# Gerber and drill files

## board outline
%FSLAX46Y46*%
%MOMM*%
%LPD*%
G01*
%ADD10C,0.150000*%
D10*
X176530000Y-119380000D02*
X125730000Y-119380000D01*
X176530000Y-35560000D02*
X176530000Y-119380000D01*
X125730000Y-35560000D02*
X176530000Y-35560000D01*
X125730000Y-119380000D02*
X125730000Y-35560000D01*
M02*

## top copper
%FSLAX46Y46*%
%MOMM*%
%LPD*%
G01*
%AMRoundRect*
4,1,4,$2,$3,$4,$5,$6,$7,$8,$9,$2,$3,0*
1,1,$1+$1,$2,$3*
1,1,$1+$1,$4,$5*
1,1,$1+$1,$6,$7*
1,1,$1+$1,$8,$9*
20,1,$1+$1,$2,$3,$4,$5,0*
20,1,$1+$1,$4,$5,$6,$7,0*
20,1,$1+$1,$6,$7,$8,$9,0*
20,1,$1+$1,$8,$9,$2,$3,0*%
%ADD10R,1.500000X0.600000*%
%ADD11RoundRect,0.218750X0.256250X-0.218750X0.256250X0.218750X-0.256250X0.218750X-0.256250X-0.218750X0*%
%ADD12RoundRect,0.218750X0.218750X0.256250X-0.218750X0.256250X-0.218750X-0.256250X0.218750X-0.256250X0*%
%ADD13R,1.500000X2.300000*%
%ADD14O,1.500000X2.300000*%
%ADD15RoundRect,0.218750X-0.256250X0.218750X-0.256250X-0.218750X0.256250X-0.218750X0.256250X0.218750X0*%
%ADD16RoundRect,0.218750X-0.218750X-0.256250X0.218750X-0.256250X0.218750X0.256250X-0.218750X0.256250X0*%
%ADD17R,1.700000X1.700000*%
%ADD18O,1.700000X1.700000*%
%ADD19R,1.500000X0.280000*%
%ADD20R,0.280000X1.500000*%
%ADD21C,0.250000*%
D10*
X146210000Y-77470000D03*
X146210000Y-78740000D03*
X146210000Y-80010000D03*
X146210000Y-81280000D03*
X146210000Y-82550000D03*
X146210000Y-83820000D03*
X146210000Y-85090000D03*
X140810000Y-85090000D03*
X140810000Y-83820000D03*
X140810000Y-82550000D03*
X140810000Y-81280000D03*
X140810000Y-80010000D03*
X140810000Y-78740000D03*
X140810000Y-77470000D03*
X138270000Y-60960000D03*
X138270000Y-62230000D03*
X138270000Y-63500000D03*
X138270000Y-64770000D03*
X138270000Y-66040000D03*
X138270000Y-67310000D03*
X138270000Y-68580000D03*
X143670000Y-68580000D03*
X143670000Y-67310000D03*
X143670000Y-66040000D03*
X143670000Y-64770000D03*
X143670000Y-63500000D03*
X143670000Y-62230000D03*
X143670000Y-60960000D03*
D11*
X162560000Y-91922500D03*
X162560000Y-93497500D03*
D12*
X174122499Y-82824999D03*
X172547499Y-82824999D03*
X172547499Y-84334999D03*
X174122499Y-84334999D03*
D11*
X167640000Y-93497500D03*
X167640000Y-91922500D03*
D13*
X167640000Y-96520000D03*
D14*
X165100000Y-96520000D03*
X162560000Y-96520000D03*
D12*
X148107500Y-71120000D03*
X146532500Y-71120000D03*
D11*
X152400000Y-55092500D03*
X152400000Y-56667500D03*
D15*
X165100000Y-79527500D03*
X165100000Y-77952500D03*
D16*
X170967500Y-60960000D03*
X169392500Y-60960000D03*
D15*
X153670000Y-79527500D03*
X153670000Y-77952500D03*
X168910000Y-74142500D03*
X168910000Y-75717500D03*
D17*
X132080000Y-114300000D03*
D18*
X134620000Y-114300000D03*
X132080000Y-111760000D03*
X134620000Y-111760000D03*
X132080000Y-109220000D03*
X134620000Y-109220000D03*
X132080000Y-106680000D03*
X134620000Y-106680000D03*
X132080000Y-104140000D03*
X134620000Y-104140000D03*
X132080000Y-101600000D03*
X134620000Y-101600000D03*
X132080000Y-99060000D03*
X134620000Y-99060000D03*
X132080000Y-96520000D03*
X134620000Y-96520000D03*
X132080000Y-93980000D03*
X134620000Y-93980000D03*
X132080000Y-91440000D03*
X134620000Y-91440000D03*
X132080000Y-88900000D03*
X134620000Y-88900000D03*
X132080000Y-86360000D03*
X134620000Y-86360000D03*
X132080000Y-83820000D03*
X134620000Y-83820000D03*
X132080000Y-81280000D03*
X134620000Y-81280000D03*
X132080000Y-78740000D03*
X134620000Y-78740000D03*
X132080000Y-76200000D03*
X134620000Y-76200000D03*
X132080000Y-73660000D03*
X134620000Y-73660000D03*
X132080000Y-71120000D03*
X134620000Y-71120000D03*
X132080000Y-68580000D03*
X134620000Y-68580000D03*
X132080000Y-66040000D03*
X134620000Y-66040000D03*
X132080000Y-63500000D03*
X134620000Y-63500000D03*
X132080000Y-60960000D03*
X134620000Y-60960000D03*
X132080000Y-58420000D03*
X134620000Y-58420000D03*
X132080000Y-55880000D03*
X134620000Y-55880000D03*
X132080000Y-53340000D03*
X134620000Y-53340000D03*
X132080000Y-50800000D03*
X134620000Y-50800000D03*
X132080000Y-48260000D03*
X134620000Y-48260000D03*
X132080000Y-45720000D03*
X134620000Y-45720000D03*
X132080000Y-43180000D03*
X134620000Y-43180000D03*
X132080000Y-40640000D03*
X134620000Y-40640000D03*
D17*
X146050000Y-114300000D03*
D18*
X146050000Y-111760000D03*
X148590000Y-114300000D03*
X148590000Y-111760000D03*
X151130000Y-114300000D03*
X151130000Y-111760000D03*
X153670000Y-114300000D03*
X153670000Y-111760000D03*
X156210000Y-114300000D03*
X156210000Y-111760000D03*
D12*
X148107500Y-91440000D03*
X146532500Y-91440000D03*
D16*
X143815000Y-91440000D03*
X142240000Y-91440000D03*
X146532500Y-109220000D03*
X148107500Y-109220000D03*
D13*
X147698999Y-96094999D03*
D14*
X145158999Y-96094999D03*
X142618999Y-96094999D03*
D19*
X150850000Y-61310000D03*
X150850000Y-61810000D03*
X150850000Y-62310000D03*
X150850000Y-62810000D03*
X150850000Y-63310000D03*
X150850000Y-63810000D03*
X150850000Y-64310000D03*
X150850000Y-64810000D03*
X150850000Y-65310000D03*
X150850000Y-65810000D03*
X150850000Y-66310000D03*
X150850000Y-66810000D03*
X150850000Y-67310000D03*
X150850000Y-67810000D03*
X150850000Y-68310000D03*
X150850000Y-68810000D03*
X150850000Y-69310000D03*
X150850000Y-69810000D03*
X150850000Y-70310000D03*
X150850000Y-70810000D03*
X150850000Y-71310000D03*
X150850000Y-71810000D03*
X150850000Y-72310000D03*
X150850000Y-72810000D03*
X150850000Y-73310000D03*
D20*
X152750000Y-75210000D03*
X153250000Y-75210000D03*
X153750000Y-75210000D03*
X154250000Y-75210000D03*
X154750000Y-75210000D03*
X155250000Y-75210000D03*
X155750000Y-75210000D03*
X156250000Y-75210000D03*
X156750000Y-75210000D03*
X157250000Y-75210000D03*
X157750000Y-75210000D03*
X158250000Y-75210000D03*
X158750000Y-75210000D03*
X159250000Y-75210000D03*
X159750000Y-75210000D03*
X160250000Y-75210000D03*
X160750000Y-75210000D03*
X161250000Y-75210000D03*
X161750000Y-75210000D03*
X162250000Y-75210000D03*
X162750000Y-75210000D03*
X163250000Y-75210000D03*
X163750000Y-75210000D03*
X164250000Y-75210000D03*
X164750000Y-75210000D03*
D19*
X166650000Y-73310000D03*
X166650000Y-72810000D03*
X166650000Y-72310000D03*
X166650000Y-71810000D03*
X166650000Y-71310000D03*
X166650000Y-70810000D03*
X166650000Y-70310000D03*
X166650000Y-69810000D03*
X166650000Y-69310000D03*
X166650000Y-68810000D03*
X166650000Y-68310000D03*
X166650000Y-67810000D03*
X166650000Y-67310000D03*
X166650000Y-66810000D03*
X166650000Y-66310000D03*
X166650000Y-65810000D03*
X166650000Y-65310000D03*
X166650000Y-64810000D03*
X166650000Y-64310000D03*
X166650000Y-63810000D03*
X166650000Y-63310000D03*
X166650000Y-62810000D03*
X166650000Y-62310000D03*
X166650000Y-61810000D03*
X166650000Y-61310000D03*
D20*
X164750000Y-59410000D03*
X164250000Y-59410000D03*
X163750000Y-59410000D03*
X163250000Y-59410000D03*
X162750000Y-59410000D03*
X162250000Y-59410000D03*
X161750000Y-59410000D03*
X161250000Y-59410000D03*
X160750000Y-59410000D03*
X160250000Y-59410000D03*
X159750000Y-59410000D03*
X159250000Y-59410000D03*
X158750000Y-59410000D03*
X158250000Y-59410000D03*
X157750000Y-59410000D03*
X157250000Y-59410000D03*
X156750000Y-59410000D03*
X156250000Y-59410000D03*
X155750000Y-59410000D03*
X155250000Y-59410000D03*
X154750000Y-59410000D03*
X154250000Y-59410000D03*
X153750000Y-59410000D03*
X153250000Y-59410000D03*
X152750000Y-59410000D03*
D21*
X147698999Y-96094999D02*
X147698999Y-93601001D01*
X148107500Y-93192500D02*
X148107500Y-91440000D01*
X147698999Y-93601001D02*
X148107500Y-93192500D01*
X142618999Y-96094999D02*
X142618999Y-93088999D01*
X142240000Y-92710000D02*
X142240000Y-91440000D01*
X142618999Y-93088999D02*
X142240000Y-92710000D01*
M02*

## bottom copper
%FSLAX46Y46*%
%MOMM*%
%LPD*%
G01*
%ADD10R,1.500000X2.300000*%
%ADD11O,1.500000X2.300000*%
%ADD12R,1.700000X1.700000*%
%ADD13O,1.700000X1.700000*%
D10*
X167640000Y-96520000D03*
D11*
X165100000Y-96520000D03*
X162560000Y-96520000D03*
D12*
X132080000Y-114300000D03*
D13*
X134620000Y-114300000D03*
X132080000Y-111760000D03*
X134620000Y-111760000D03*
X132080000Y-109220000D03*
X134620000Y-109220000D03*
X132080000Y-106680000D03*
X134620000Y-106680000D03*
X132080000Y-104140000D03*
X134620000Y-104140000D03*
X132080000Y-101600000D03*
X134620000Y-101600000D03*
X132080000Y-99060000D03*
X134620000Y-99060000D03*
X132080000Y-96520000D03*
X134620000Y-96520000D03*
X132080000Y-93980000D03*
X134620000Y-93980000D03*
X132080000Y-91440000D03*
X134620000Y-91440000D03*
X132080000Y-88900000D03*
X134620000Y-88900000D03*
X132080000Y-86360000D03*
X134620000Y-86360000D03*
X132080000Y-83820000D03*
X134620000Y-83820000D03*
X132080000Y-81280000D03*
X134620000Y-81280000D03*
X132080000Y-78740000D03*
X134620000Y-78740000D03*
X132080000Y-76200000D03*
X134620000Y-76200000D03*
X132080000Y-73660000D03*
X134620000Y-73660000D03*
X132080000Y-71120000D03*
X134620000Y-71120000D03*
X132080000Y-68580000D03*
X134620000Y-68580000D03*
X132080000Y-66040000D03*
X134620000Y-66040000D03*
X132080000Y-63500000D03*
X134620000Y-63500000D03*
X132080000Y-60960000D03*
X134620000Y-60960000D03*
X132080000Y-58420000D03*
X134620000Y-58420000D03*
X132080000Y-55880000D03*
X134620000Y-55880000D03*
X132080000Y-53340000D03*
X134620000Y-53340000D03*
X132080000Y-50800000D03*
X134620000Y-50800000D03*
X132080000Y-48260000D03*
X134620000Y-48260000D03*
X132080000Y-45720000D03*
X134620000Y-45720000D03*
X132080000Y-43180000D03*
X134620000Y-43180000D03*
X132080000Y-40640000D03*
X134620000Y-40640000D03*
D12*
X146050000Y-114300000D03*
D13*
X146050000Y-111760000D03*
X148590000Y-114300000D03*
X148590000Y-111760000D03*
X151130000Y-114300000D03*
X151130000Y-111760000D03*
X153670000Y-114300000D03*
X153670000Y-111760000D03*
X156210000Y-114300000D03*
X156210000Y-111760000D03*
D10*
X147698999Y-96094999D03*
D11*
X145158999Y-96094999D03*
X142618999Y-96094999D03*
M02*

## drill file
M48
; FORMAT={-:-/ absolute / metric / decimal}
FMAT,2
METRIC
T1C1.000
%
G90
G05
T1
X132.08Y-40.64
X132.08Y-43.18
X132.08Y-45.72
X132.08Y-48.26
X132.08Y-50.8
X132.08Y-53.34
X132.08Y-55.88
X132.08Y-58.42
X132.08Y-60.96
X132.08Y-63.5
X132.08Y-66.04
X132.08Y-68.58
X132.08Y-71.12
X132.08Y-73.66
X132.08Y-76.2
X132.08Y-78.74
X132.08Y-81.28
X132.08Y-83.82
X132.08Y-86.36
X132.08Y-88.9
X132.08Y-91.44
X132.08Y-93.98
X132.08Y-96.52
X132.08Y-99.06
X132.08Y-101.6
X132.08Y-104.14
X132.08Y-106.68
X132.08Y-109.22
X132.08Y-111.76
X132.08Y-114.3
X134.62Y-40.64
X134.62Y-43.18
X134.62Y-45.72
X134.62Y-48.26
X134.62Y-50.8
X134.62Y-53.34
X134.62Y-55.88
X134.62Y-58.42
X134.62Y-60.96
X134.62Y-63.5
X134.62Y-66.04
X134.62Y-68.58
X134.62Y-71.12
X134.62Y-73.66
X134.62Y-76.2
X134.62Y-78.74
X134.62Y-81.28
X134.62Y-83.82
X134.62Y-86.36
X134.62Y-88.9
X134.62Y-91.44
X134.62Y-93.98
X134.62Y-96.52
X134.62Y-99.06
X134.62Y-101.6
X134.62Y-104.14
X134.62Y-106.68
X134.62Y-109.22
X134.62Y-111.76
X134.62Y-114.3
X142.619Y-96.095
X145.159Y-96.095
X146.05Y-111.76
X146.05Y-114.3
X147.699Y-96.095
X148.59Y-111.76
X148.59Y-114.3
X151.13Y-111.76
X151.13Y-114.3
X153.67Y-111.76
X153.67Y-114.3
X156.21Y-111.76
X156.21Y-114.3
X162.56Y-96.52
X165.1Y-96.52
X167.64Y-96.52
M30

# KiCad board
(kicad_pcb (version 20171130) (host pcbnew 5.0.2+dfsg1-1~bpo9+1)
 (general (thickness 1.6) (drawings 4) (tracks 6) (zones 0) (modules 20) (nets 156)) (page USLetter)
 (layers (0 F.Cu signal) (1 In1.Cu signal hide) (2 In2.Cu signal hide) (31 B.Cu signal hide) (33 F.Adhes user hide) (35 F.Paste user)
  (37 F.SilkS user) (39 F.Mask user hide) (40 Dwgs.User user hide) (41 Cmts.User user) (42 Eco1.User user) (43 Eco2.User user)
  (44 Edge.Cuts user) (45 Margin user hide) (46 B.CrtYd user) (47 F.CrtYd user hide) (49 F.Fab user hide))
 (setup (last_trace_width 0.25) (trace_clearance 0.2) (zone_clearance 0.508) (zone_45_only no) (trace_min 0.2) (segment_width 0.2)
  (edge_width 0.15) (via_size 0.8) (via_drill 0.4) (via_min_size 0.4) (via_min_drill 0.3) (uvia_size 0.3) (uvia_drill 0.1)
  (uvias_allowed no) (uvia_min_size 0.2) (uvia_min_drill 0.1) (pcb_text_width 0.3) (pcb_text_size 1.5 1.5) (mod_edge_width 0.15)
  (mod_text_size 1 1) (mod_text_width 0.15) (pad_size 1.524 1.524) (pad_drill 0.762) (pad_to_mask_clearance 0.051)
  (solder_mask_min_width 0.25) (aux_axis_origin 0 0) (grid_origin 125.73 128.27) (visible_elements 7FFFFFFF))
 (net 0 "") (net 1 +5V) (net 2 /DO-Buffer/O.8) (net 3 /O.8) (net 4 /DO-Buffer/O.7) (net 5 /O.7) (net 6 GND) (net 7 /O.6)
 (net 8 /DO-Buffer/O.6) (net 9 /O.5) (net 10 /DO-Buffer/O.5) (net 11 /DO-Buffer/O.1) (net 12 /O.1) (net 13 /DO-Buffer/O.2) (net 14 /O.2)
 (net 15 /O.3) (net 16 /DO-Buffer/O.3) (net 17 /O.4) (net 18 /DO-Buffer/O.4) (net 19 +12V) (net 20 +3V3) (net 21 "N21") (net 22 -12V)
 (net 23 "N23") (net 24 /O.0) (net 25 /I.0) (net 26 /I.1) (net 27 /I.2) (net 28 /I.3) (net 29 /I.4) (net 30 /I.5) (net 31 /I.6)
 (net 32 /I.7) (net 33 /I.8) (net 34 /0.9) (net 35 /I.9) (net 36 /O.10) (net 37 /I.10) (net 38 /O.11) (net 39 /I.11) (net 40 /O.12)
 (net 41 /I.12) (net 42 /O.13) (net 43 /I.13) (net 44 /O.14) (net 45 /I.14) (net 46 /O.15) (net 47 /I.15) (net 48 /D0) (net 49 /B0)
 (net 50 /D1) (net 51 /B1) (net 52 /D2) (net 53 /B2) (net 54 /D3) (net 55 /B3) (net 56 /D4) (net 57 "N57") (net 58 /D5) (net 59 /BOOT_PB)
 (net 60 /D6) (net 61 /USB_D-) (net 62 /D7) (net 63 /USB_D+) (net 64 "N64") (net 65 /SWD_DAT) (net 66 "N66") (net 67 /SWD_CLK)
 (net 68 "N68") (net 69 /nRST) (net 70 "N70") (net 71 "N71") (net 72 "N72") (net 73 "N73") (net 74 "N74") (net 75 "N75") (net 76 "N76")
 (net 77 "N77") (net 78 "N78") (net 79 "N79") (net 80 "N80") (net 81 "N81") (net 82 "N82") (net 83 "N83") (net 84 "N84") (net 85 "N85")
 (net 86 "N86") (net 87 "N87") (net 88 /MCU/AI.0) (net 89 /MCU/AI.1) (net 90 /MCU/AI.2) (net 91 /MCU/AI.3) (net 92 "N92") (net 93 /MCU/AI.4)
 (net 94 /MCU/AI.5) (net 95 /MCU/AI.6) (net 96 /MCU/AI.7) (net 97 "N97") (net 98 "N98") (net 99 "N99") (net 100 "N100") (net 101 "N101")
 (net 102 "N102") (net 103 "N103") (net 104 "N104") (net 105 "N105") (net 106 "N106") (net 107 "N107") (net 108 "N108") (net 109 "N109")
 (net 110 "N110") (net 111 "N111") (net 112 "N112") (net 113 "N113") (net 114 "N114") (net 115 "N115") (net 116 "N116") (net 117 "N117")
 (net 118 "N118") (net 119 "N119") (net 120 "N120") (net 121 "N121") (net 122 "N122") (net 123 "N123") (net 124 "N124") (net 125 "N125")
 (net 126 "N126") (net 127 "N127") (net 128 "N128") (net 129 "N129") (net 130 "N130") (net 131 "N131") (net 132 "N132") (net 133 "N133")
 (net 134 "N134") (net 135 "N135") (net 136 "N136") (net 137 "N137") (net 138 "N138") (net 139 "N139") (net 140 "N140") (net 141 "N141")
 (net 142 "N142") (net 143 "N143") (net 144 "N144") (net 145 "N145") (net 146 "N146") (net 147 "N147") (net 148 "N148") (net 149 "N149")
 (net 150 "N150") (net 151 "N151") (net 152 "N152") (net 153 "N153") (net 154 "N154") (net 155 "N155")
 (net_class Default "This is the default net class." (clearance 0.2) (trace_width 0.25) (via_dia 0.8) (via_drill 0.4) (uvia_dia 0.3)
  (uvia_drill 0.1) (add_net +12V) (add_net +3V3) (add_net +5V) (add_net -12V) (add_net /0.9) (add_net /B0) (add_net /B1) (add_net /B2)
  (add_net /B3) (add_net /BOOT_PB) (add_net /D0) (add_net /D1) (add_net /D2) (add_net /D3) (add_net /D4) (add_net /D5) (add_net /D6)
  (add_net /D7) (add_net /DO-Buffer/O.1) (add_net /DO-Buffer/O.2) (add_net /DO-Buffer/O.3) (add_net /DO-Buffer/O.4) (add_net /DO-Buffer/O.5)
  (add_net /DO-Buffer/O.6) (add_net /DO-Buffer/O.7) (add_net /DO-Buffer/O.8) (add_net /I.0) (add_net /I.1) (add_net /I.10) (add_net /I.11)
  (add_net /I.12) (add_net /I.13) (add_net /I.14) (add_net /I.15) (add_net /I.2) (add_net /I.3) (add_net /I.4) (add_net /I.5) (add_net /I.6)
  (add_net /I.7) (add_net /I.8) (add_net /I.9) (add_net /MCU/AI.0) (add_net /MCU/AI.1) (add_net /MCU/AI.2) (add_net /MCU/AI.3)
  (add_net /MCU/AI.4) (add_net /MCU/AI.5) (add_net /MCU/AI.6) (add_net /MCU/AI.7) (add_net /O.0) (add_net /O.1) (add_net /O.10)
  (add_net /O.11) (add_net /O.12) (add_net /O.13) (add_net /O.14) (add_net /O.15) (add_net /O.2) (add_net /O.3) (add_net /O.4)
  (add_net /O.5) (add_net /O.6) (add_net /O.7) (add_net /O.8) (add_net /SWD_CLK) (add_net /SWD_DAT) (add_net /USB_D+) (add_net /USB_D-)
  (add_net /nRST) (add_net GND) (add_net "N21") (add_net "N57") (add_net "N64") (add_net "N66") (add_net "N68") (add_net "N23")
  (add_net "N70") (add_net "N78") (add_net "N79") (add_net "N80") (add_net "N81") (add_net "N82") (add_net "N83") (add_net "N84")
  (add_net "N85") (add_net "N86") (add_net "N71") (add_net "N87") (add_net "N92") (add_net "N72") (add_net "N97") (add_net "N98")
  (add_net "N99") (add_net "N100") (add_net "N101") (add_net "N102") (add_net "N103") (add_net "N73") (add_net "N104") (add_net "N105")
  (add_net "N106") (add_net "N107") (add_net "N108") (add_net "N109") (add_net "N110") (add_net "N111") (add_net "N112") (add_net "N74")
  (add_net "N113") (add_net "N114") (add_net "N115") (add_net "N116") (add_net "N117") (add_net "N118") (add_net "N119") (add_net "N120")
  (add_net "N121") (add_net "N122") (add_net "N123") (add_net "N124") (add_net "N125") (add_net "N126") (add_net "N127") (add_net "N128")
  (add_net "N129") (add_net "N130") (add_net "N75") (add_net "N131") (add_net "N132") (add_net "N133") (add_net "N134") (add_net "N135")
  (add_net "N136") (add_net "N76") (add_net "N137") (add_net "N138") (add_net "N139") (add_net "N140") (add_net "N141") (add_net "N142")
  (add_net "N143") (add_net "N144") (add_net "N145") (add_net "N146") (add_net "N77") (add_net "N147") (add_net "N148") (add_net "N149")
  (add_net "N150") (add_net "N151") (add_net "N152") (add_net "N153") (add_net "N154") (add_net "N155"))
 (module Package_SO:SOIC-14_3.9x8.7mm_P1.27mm (layer F.Cu) (at 143.51 81.28)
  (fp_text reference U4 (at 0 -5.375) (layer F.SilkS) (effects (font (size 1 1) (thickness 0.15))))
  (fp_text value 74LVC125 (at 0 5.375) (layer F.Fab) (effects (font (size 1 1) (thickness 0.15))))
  (pad 14 smd rect (at 2.7 -3.81) (size 1.5 0.6) (layers F.Cu F.Paste F.Mask) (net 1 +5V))
  (pad 13 smd rect (at 2.7 -2.54) (size 1.5 0.6) (layers F.Cu F.Paste F.Mask) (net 1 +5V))
  (pad 12 smd rect (at 2.7 -1.27) (size 1.5 0.6) (layers F.Cu F.Paste F.Mask) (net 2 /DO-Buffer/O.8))
  (pad 11 smd rect (at 2.7 0) (size 1.5 0.6) (layers F.Cu F.Paste F.Mask) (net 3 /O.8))
  (pad 10 smd rect (at 2.7 1.27) (size 1.5 0.6) (layers F.Cu F.Paste F.Mask) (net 1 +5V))
  (pad 9 smd rect (at 2.7 2.54) (size 1.5 0.6) (layers F.Cu F.Paste F.Mask) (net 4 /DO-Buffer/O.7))
  (pad 8 smd rect (at 2.7 3.81) (size 1.5 0.6) (layers F.Cu F.Paste F.Mask) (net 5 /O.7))
  (pad 7 smd rect (at -2.7 3.81) (size 1.5 0.6) (layers F.Cu F.Paste F.Mask) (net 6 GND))
  (pad 6 smd rect (at -2.7 2.54) (size 1.5 0.6) (layers F.Cu F.Paste F.Mask) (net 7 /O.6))
  (pad 5 smd rect (at -2.7 1.27) (size 1.5 0.6) (layers F.Cu F.Paste F.Mask) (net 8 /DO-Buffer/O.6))
  (pad 4 smd rect (at -2.7 0) (size 1.5 0.6) (layers F.Cu F.Paste F.Mask) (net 1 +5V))
  (pad 3 smd rect (at -2.7 -1.27) (size 1.5 0.6) (layers F.Cu F.Paste F.Mask) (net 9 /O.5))
  (pad 2 smd rect (at -2.7 -2.54) (size 1.5 0.6) (layers F.Cu F.Paste F.Mask) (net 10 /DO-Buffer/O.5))
  (pad 1 smd rect (at -2.7 -3.81) (size 1.5 0.6) (layers F.Cu F.Paste F.Mask) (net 1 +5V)))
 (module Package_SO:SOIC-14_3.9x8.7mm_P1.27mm (layer F.Cu) (at 140.97 64.77)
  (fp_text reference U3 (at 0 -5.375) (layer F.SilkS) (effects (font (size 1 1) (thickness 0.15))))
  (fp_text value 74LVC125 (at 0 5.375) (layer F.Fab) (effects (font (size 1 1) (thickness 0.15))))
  (pad 1 smd rect (at -2.7 -3.81) (size 1.5 0.6) (layers F.Cu F.Paste F.Mask) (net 1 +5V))
  (pad 2 smd rect (at -2.7 -2.54) (size 1.5 0.6) (layers F.Cu F.Paste F.Mask) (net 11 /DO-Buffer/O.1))
  (pad 3 smd rect (at -2.7 -1.27) (size 1.5 0.6) (layers F.Cu F.Paste F.Mask) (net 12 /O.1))
  (pad 4 smd rect (at -2.7 0) (size 1.5 0.6) (layers F.Cu F.Paste F.Mask) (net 1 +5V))
  (pad 5 smd rect (at -2.7 1.27) (size 1.5 0.6) (layers F.Cu F.Paste F.Mask) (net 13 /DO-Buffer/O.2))
  (pad 6 smd rect (at -2.7 2.54) (size 1.5 0.6) (layers F.Cu F.Paste F.Mask) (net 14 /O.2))
  (pad 7 smd rect (at -2.7 3.81) (size 1.5 0.6) (layers F.Cu F.Paste F.Mask) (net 6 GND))
  (pad 8 smd rect (at 2.7 3.81) (size 1.5 0.6) (layers F.Cu F.Paste F.Mask) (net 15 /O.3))
  (pad 9 smd rect (at 2.7 2.54) (size 1.5 0.6) (layers F.Cu F.Paste F.Mask) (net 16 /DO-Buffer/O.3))
  (pad 10 smd rect (at 2.7 1.27) (size 1.5 0.6) (layers F.Cu F.Paste F.Mask) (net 1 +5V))
  (pad 11 smd rect (at 2.7 0) (size 1.5 0.6) (layers F.Cu F.Paste F.Mask) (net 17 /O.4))
  (pad 12 smd rect (at 2.7 -1.27) (size 1.5 0.6) (layers F.Cu F.Paste F.Mask) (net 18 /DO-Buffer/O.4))
  (pad 13 smd rect (at 2.7 -2.54) (size 1.5 0.6) (layers F.Cu F.Paste F.Mask) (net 1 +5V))
  (pad 14 smd rect (at 2.7 -3.81) (size 1.5 0.6) (layers F.Cu F.Paste F.Mask) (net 1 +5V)))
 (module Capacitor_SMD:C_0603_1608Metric (layer F.Cu) (at 162.56 92.71 90)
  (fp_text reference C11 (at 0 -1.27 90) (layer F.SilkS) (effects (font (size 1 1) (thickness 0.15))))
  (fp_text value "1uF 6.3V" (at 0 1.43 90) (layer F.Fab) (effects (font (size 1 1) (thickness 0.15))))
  (pad 2 smd roundrect (at 0.7875 0 90) (size 0.875 0.95) (layers F.Cu F.Paste F.Mask) (roundrect_rratio 0.25) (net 6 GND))
  (pad 1 smd roundrect (at -0.7875 0 90) (size 0.875 0.95) (layers F.Cu F.Paste F.Mask) (roundrect_rratio 0.25) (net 1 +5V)))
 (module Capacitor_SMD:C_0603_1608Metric (layer F.Cu) (at 173.334999 82.824999 180)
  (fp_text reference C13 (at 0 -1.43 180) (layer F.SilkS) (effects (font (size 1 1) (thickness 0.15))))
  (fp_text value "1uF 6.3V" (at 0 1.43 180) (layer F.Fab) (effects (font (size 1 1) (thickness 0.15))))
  (pad 1 smd roundrect (at -0.7875 0 180) (size 0.875 0.95) (layers F.Cu F.Paste F.Mask) (roundrect_rratio 0.25) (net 1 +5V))
  (pad 2 smd roundrect (at 0.7875 0 180) (size 0.875 0.95) (layers F.Cu F.Paste F.Mask) (roundrect_rratio 0.25) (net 6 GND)))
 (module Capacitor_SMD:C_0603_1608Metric (layer F.Cu) (at 173.334999 84.334999 180)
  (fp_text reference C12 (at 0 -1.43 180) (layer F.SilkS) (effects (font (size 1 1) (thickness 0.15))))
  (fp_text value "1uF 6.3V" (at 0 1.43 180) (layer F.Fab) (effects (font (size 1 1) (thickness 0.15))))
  (pad 2 smd roundrect (at 0.7875 0 180) (size 0.875 0.95) (layers F.Cu F.Paste F.Mask) (roundrect_rratio 0.25) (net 6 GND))
  (pad 1 smd roundrect (at -0.7875 0 180) (size 0.875 0.95) (layers F.Cu F.Paste F.Mask) (roundrect_rratio 0.25) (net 1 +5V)))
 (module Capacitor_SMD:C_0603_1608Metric (layer F.Cu) (at 167.64 92.71 90)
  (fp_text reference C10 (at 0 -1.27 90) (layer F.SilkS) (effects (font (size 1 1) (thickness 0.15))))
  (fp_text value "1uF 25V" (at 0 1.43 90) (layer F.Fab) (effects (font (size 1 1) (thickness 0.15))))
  (pad 1 smd roundrect (at -0.7875 0 90) (size 0.875 0.95) (layers F.Cu F.Paste F.Mask) (roundrect_rratio 0.25) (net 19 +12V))
  (pad 2 smd roundrect (at 0.7875 0 90) (size 0.875 0.95) (layers F.Cu F.Paste F.Mask) (roundrect_rratio 0.25) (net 6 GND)))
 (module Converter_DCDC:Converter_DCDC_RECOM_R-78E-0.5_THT (layer F.Cu) (at 167.64 96.52 180)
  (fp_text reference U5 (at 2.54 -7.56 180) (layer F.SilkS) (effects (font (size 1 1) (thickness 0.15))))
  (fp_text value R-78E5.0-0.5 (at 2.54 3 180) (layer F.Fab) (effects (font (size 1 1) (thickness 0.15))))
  (pad 1 thru_hole rect (at 0 0 180) (size 1.5 2.3) (drill 1) (layers *.Cu *.Mask) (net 19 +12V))
  (pad 2 thru_hole oval (at 2.54 0 180) (size 1.5 2.3) (drill 1) (layers *.Cu *.Mask) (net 6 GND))
  (pad 3 thru_hole oval (at 5.08 0 180) (size 1.5 2.3) (drill 1) (layers *.Cu *.Mask) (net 1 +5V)))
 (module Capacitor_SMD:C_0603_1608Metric (layer F.Cu) (at 147.32 71.12 180)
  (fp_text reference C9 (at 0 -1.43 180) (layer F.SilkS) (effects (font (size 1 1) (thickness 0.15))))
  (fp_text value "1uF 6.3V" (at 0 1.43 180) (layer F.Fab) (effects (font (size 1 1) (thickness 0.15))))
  (pad 1 smd roundrect (at -0.7875 0 180) (size 0.875 0.95) (layers F.Cu F.Paste F.Mask) (roundrect_rratio 0.25) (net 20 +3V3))
  (pad 2 smd roundrect (at 0.7875 0 180) (size 0.875 0.95) (layers F.Cu F.Paste F.Mask) (roundrect_rratio 0.25) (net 6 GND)))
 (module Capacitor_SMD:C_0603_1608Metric (layer F.Cu) (at 152.4 55.88 90)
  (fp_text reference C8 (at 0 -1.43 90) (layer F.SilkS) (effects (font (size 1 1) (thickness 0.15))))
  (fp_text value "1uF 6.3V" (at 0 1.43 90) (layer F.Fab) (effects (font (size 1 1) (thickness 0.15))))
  (pad 2 smd roundrect (at 0.7875 0 90) (size 0.875 0.95) (layers F.Cu F.Paste F.Mask) (roundrect_rratio 0.25) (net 6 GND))
  (pad 1 smd roundrect (at -0.7875 0 90) (size 0.875 0.95) (layers F.Cu F.Paste F.Mask) (roundrect_rratio 0.25) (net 20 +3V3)))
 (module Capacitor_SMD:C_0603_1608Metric (layer F.Cu) (at 165.1 78.74 270)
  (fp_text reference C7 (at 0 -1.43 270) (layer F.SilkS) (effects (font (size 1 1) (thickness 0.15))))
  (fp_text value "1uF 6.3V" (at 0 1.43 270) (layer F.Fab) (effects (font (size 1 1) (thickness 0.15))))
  (pad 2 smd roundrect (at 0.7875 0 270) (size 0.875 0.95) (layers F.Cu F.Paste F.Mask) (roundrect_rratio 0.25) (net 6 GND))
  (pad 1 smd roundrect (at -0.7875 0 270) (size 0.875 0.95) (layers F.Cu F.Paste F.Mask) (roundrect_rratio 0.25) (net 20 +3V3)))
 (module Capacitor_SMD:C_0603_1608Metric (layer F.Cu) (at 170.18 60.96)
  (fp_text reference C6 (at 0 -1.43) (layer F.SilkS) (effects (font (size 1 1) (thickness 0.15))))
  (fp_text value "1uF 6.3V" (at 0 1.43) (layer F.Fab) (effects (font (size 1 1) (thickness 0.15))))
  (pad 2 smd roundrect (at 0.7875 0) (size 0.875 0.95) (layers F.Cu F.Paste F.Mask) (roundrect_rratio 0.25) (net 6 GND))
  (pad 1 smd roundrect (at -0.7875 0) (size 0.875 0.95) (layers F.Cu F.Paste F.Mask) (roundrect_rratio 0.25) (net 20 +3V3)))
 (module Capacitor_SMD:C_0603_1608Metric (layer F.Cu) (at 153.67 78.74 270)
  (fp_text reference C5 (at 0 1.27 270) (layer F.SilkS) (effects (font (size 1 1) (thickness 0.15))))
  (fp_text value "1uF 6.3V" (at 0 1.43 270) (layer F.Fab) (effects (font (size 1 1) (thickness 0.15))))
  (pad 2 smd roundrect (at 0.7875 0 270) (size 0.875 0.95) (layers F.Cu F.Paste F.Mask) (roundrect_rratio 0.25) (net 6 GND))
  (pad 1 smd roundrect (at -0.7875 0 270) (size 0.875 0.95) (layers F.Cu F.Paste F.Mask) (roundrect_rratio 0.25) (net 20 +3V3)))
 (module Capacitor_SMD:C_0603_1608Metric (layer F.Cu) (at 168.91 74.93 270)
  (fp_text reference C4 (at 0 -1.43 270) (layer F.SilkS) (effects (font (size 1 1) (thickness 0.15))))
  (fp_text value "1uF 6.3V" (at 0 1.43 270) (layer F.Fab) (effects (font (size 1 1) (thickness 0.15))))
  (pad 1 smd roundrect (at -0.7875 0 270) (size 0.875 0.95) (layers F.Cu F.Paste F.Mask) (roundrect_rratio 0.25) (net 20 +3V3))
  (pad 2 smd roundrect (at 0.7875 0 270) (size 0.875 0.95) (layers F.Cu F.Paste F.Mask) (roundrect_rratio 0.25) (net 6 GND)))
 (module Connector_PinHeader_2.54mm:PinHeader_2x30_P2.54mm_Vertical (layer B.Cu) (at 132.08 114.3)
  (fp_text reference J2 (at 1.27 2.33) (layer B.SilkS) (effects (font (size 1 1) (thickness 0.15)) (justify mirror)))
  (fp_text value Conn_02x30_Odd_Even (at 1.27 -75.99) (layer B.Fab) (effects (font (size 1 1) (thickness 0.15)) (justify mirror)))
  (pad 1 thru_hole rect (at 0 0) (size 1.7 1.7) (drill 1) (layers *.Cu *.Mask) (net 20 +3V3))
  (pad 2 thru_hole oval (at 2.54 0) (size 1.7 1.7) (drill 1) (layers *.Cu *.Mask) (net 6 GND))
  (pad 3 thru_hole oval (at 0 -2.54) (size 1.7 1.7) (drill 1) (layers *.Cu *.Mask) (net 19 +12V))
  (pad 4 thru_hole oval (at 2.54 -2.54) (size 1.7 1.7) (drill 1) (layers *.Cu *.Mask) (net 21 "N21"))
  (pad 5 thru_hole oval (at 0 -5.08) (size 1.7 1.7) (drill 1) (layers *.Cu *.Mask) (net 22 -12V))
  (pad 6 thru_hole oval (at 2.54 -5.08) (size 1.7 1.7) (drill 1) (layers *.Cu *.Mask) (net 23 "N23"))
  (pad 7 thru_hole oval (at 0 -7.62) (size 1.7 1.7) (drill 1) (layers *.Cu *.Mask) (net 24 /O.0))
  (pad 8 thru_hole oval (at 2.54 -7.62) (size 1.7 1.7) (drill 1) (layers *.Cu *.Mask) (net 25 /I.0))
  (pad 9 thru_hole oval (at 0 -10.16) (size 1.7 1.7) (drill 1) (layers *.Cu *.Mask) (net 12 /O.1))
  (pad 10 thru_hole oval (at 2.54 -10.16) (size 1.7 1.7) (drill 1) (layers *.Cu *.Mask) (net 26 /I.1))
  (pad 11 thru_hole oval (at 0 -12.7) (size 1.7 1.7) (drill 1) (layers *.Cu *.Mask) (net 14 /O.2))
  (pad 12 thru_hole oval (at 2.54 -12.7) (size 1.7 1.7) (drill 1) (layers *.Cu *.Mask) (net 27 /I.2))
  (pad 13 thru_hole oval (at 0 -15.24) (size 1.7 1.7) (drill 1) (layers *.Cu *.Mask) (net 15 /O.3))
  (pad 14 thru_hole oval (at 2.54 -15.24) (size 1.7 1.7) (drill 1) (layers *.Cu *.Mask) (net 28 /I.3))
  (pad 15 thru_hole oval (at 0 -17.78) (size 1.7 1.7) (drill 1) (layers *.Cu *.Mask) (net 17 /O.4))
  (pad 16 thru_hole oval (at 2.54 -17.78) (size 1.7 1.7) (drill 1) (layers *.Cu *.Mask) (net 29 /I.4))
  (pad 17 thru_hole oval (at 0 -20.32) (size 1.7 1.7) (drill 1) (layers *.Cu *.Mask) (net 9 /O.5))
  (pad 18 thru_hole oval (at 2.54 -20.32) (size 1.7 1.7) (drill 1) (layers *.Cu *.Mask) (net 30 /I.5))
  (pad 19 thru_hole oval (at 0 -22.86) (size 1.7 1.7) (drill 1) (layers *.Cu *.Mask) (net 7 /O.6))
  (pad 20 thru_hole oval (at 2.54 -22.86) (size 1.7 1.7) (drill 1) (layers *.Cu *.Mask) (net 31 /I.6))
  (pad 21 thru_hole oval (at 0 -25.4) (size 1.7 1.7) (drill 1) (layers *.Cu *.Mask) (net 5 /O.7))
  (pad 22 thru_hole oval (at 2.54 -25.4) (size 1.7 1.7) (drill 1) (layers *.Cu *.Mask) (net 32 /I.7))
  (pad 23 thru_hole oval (at 0 -27.94) (size 1.7 1.7) (drill 1) (layers *.Cu *.Mask) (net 3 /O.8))
  (pad 24 thru_hole oval (at 2.54 -27.94) (size 1.7 1.7) (drill 1) (layers *.Cu *.Mask) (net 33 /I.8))
  (pad 25 thru_hole oval (at 0 -30.48) (size 1.7 1.7) (drill 1) (layers *.Cu *.Mask) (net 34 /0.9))
  (pad 26 thru_hole oval (at 2.54 -30.48) (size 1.7 1.7) (drill 1) (layers *.Cu *.Mask) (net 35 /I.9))
  (pad 27 thru_hole oval (at 0 -33.02) (size 1.7 1.7) (drill 1) (layers *.Cu *.Mask) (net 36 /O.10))
  (pad 28 thru_hole oval (at 2.54 -33.02) (size 1.7 1.7) (drill 1) (layers *.Cu *.Mask) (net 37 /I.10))
  (pad 29 thru_hole oval (at 0 -35.56) (size 1.7 1.7) (drill 1) (layers *.Cu *.Mask) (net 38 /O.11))
  (pad 30 thru_hole oval (at 2.54 -35.56) (size 1.7 1.7) (drill 1) (layers *.Cu *.Mask) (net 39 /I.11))
  (pad 31 thru_hole oval (at 0 -38.1) (size 1.7 1.7) (drill 1) (layers *.Cu *.Mask) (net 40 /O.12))
  (pad 32 thru_hole oval (at 2.54 -38.1) (size 1.7 1.7) (drill 1) (layers *.Cu *.Mask) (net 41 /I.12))
  (pad 33 thru_hole oval (at 0 -40.64) (size 1.7 1.7) (drill 1) (layers *.Cu *.Mask) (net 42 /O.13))
  (pad 34 thru_hole oval (at 2.54 -40.64) (size 1.7 1.7) (drill 1) (layers *.Cu *.Mask) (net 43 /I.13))
  (pad 35 thru_hole oval (at 0 -43.18) (size 1.7 1.7) (drill 1) (layers *.Cu *.Mask) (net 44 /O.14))
  (pad 36 thru_hole oval (at 2.54 -43.18) (size 1.7 1.7) (drill 1) (layers *.Cu *.Mask) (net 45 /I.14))
  (pad 37 thru_hole oval (at 0 -45.72) (size 1.7 1.7) (drill 1) (layers *.Cu *.Mask) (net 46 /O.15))
  (pad 38 thru_hole oval (at 2.54 -45.72) (size 1.7 1.7) (drill 1) (layers *.Cu *.Mask) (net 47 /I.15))
  (pad 39 thru_hole oval (at 0 -48.26) (size 1.7 1.7) (drill 1) (layers *.Cu *.Mask) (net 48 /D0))
  (pad 40 thru_hole oval (at 2.54 -48.26) (size 1.7 1.7) (drill 1) (layers *.Cu *.Mask) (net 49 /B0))
  (pad 41 thru_hole oval (at 0 -50.8) (size 1.7 1.7) (drill 1) (layers *.Cu *.Mask) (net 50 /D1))
  (pad 42 thru_hole oval (at 2.54 -50.8) (size 1.7 1.7) (drill 1) (layers *.Cu *.Mask) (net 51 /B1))
  (pad 43 thru_hole oval (at 0 -53.34) (size 1.7 1.7) (drill 1) (layers *.Cu *.Mask) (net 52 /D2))
  (pad 44 thru_hole oval (at 2.54 -53.34) (size 1.7 1.7) (drill 1) (layers *.Cu *.Mask) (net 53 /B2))
  (pad 45 thru_hole oval (at 0 -55.88) (size 1.7 1.7) (drill 1) (layers *.Cu *.Mask) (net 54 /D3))
  (pad 46 thru_hole oval (at 2.54 -55.88) (size 1.7 1.7) (drill 1) (layers *.Cu *.Mask) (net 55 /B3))
  (pad 47 thru_hole oval (at 0 -58.42) (size 1.7 1.7) (drill 1) (layers *.Cu *.Mask) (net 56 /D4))
  (pad 48 thru_hole oval (at 2.54 -58.42) (size 1.7 1.7) (drill 1) (layers *.Cu *.Mask) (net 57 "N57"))
  (pad 49 thru_hole oval (at 0 -60.96) (size 1.7 1.7) (drill 1) (layers *.Cu *.Mask) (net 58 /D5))
  (pad 50 thru_hole oval (at 2.54 -60.96) (size 1.7 1.7) (drill 1) (layers *.Cu *.Mask) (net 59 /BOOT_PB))
  (pad 51 thru_hole oval (at 0 -63.5) (size 1.7 1.7) (drill 1) (layers *.Cu *.Mask) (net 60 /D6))
  (pad 52 thru_hole oval (at 2.54 -63.5) (size 1.7 1.7) (drill 1) (layers *.Cu *.Mask) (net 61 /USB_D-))
  (pad 53 thru_hole oval (at 0 -66.04) (size 1.7 1.7) (drill 1) (layers *.Cu *.Mask) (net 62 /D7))
  (pad 54 thru_hole oval (at 2.54 -66.04) (size 1.7 1.7) (drill 1) (layers *.Cu *.Mask) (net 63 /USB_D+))
  (pad 55 thru_hole oval (at 0 -68.58) (size 1.7 1.7) (drill 1) (layers *.Cu *.Mask) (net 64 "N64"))
  (pad 56 thru_hole oval (at 2.54 -68.58) (size 1.7 1.7) (drill 1) (layers *.Cu *.Mask) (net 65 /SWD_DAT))
  (pad 57 thru_hole oval (at 0 -71.12) (size 1.7 1.7) (drill 1) (layers *.Cu *.Mask) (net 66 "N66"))
  (pad 58 thru_hole oval (at 2.54 -71.12) (size 1.7 1.7) (drill 1) (layers *.Cu *.Mask) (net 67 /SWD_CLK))
  (pad 59 thru_hole oval (at 0 -73.66) (size 1.7 1.7) (drill 1) (layers *.Cu *.Mask) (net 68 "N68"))
  (pad 60 thru_hole oval (at 2.54 -73.66) (size 1.7 1.7) (drill 1) (layers *.Cu *.Mask) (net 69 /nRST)))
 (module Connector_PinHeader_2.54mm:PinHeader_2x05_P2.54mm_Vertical (layer F.Cu) (at 146.05 114.3 90)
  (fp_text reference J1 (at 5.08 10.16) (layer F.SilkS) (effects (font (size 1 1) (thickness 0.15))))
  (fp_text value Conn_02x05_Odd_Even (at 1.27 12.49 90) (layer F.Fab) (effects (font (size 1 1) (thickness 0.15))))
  (pad 1 thru_hole rect (at 0 0 90) (size 1.7 1.7) (drill 1) (layers *.Cu *.Mask) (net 19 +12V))
  (pad 2 thru_hole oval (at 2.54 0 90) (size 1.7 1.7) (drill 1) (layers *.Cu *.Mask) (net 19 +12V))
  (pad 3 thru_hole oval (at 0 2.54 90) (size 1.7 1.7) (drill 1) (layers *.Cu *.Mask) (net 6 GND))
  (pad 4 thru_hole oval (at 2.54 2.54 90) (size 1.7 1.7) (drill 1) (layers *.Cu *.Mask) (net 6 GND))
  (pad 5 thru_hole oval (at 0 5.08 90) (size 1.7 1.7) (drill 1) (layers *.Cu *.Mask) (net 6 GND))
  (pad 6 thru_hole oval (at 2.54 5.08 90) (size 1.7 1.7) (drill 1) (layers *.Cu *.Mask) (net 6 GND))
  (pad 7 thru_hole oval (at 0 7.62 90) (size 1.7 1.7) (drill 1) (layers *.Cu *.Mask) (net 6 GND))
  (pad 8 thru_hole oval (at 2.54 7.62 90) (size 1.7 1.7) (drill 1) (layers *.Cu *.Mask) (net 6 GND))
  (pad 9 thru_hole oval (at 0 10.16 90) (size 1.7 1.7) (drill 1) (layers *.Cu *.Mask) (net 22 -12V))
  (pad 10 thru_hole oval (at 2.54 10.16 90) (size 1.7 1.7) (drill 1) (layers *.Cu *.Mask) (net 22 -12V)))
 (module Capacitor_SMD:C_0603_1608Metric (layer F.Cu) (at 147.32 91.44 180)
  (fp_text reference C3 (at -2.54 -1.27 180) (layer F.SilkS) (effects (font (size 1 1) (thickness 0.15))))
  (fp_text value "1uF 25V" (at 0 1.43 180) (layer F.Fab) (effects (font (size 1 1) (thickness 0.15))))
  (pad 1 smd roundrect (at -0.7875 0 180) (size 0.875 0.95) (layers F.Cu F.Paste F.Mask) (roundrect_rratio 0.25) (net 19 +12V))
  (pad 2 smd roundrect (at 0.7875 0 180) (size 0.875 0.95) (layers F.Cu F.Paste F.Mask) (roundrect_rratio 0.25) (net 6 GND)))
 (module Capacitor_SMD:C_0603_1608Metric (layer F.Cu) (at 143.0275 91.44)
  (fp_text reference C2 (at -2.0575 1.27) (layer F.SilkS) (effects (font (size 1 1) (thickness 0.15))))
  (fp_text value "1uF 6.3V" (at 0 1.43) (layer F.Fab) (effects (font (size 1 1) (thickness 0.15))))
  (pad 2 smd roundrect (at 0.7875 0) (size 0.875 0.95) (layers F.Cu F.Paste F.Mask) (roundrect_rratio 0.25) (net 6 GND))
  (pad 1 smd roundrect (at -0.7875 0) (size 0.875 0.95) (layers F.Cu F.Paste F.Mask) (roundrect_rratio 0.25) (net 20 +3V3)))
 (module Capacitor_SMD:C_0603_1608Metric (layer F.Cu) (at 147.32 109.22)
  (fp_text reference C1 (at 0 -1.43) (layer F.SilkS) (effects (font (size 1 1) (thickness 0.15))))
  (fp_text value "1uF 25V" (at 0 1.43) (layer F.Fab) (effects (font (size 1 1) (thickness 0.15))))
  (pad 1 smd roundrect (at -0.7875 0) (size 0.875 0.95) (layers F.Cu F.Paste F.Mask) (roundrect_rratio 0.25) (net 19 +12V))
  (pad 2 smd roundrect (at 0.7875 0) (size 0.875 0.95) (layers F.Cu F.Paste F.Mask) (roundrect_rratio 0.25) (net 6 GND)))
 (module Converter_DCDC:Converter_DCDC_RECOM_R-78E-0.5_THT (layer F.Cu) (at 147.698999 96.094999 180)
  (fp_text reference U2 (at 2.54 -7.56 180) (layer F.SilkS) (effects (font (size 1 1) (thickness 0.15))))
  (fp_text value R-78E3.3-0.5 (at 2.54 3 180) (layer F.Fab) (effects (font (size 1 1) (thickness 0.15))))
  (pad 1 thru_hole rect (at 0 0 180) (size 1.5 2.3) (drill 1) (layers *.Cu *.Mask) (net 19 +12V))
  (pad 2 thru_hole oval (at 2.54 0 180) (size 1.5 2.3) (drill 1) (layers *.Cu *.Mask) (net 6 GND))
  (pad 3 thru_hole oval (at 5.08 0 180) (size 1.5 2.3) (drill 1) (layers *.Cu *.Mask) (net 20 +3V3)))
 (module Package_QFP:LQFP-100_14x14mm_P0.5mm (layer F.Cu) (at 158.75 67.31)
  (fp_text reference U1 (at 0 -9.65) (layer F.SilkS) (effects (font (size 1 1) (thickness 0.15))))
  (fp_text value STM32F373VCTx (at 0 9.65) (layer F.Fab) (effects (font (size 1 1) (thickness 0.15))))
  (pad 1 smd rect (at -7.9 -6) (size 1.5 0.28) (layers F.Cu F.Paste F.Mask) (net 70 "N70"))
  (pad 2 smd rect (at -7.9 -5.5) (size 1.5 0.28) (layers F.Cu F.Paste F.Mask) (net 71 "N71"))
  (pad 3 smd rect (at -7.9 -5) (size 1.5 0.28) (layers F.Cu F.Paste F.Mask) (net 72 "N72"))
  (pad 4 smd rect (at -7.9 -4.5) (size 1.5 0.28) (layers F.Cu F.Paste F.Mask) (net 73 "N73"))
  (pad 5 smd rect (at -7.9 -4) (size 1.5 0.28) (layers F.Cu F.Paste F.Mask) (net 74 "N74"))
  (pad 6 smd rect (at -7.9 -3.5) (size 1.5 0.28) (layers F.Cu F.Paste F.Mask) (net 20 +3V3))
  (pad 7 smd rect (at -7.9 -3) (size 1.5 0.28) (layers F.Cu F.Paste F.Mask) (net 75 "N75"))
  (pad 8 smd rect (at -7.9 -2.5) (size 1.5 0.28) (layers F.Cu F.Paste F.Mask) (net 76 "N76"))
  (pad 9 smd rect (at -7.9 -2) (size 1.5 0.28) (layers F.Cu F.Paste F.Mask) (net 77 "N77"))
  (pad 10 smd rect (at -7.9 -1.5) (size 1.5 0.28) (layers F.Cu F.Paste F.Mask) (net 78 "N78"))
  (pad 11 smd rect (at -7.9 -1) (size 1.5 0.28) (layers F.Cu F.Paste F.Mask) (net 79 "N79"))
  (pad 12 smd rect (at -7.9 -0.5) (size 1.5 0.28) (layers F.Cu F.Paste F.Mask) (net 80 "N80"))
  (pad 13 smd rect (at -7.9 0) (size 1.5 0.28) (layers F.Cu F.Paste F.Mask) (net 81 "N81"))
  (pad 14 smd rect (at -7.9 0.5) (size 1.5 0.28) (layers F.Cu F.Paste F.Mask) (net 69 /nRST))
  (pad 15 smd rect (at -7.9 1) (size 1.5 0.28) (layers F.Cu F.Paste F.Mask) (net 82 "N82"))
  (pad 16 smd rect (at -7.9 1.5) (size 1.5 0.28) (layers F.Cu F.Paste F.Mask) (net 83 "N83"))
  (pad 17 smd rect (at -7.9 2) (size 1.5 0.28) (layers F.Cu F.Paste F.Mask) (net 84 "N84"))
  (pad 18 smd rect (at -7.9 2.5) (size 1.5 0.28) (layers F.Cu F.Paste F.Mask) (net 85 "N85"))
  (pad 19 smd rect (at -7.9 3) (size 1.5 0.28) (layers F.Cu F.Paste F.Mask) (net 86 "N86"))
  (pad 20 smd rect (at -7.9 3.5) (size 1.5 0.28) (layers F.Cu F.Paste F.Mask) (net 6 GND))
  (pad 21 smd rect (at -7.9 4) (size 1.5 0.28) (layers F.Cu F.Paste F.Mask) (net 20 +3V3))
  (pad 22 smd rect (at -7.9 4.5) (size 1.5 0.28) (layers F.Cu F.Paste F.Mask) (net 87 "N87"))
  (pad 23 smd rect (at -7.9 5) (size 1.5 0.28) (layers F.Cu F.Paste F.Mask) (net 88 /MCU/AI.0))
  (pad 24 smd rect (at -7.9 5.5) (size 1.5 0.28) (layers F.Cu F.Paste F.Mask) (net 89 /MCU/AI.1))
  (pad 25 smd rect (at -7.9 6) (size 1.5 0.28) (layers F.Cu F.Paste F.Mask) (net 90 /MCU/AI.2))
  (pad 26 smd rect (at -6 7.9 90) (size 1.5 0.28) (layers F.Cu F.Paste F.Mask) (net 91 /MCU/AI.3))
  (pad 27 smd rect (at -5.5 7.9 90) (size 1.5 0.28) (layers F.Cu F.Paste F.Mask) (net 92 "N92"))
  (pad 28 smd rect (at -5 7.9 90) (size 1.5 0.28) (layers F.Cu F.Paste F.Mask) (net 20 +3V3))
  (pad 29 smd rect (at -4.5 7.9 90) (size 1.5 0.28) (layers F.Cu F.Paste F.Mask) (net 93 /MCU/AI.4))
  (pad 30 smd rect (at -4 7.9 90) (size 1.5 0.28) (layers F.Cu F.Paste F.Mask) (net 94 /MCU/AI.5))
  (pad 31 smd rect (at -3.5 7.9 90) (size 1.5 0.28) (layers F.Cu F.Paste F.Mask) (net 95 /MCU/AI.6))
  (pad 32 smd rect (at -3 7.9 90) (size 1.5 0.28) (layers F.Cu F.Paste F.Mask) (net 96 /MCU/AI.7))
  (pad 33 smd rect (at -2.5 7.9 90) (size 1.5 0.28) (layers F.Cu F.Paste F.Mask) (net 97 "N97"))
  (pad 34 smd rect (at -2 7.9 90) (size 1.5 0.28) (layers F.Cu F.Paste F.Mask) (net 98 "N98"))
  (pad 35 smd rect (at -1.5 7.9 90) (size 1.5 0.28) (layers F.Cu F.Paste F.Mask) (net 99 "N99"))
  (pad 36 smd rect (at -1 7.9 90) (size 1.5 0.28) (layers F.Cu F.Paste F.Mask) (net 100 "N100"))
  (pad 37 smd rect (at -0.5 7.9 90) (size 1.5 0.28) (layers F.Cu F.Paste F.Mask) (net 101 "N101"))
  (pad 38 smd rect (at 0 7.9 90) (size 1.5 0.28) (layers F.Cu F.Paste F.Mask) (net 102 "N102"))
  (pad 39 smd rect (at 0.5 7.9 90) (size 1.5 0.28) (layers F.Cu F.Paste F.Mask) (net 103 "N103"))
  (pad 40 smd rect (at 1 7.9 90) (size 1.5 0.28) (layers F.Cu F.Paste F.Mask) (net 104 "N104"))
  (pad 41 smd rect (at 1.5 7.9 90) (size 1.5 0.28) (layers F.Cu F.Paste F.Mask) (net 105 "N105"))
  (pad 42 smd rect (at 2 7.9 90) (size 1.5 0.28) (layers F.Cu F.Paste F.Mask) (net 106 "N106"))
  (pad 43 smd rect (at 2.5 7.9 90) (size 1.5 0.28) (layers F.Cu F.Paste F.Mask) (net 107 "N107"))
  (pad 44 smd rect (at 3 7.9 90) (size 1.5 0.28) (layers F.Cu F.Paste F.Mask) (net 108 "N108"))
  (pad 45 smd rect (at 3.5 7.9 90) (size 1.5 0.28) (layers F.Cu F.Paste F.Mask) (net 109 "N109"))
  (pad 46 smd rect (at 4 7.9 90) (size 1.5 0.28) (layers F.Cu F.Paste F.Mask) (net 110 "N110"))
  (pad 47 smd rect (at 4.5 7.9 90) (size 1.5 0.28) (layers F.Cu F.Paste F.Mask) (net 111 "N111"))
  (pad 48 smd rect (at 5 7.9 90) (size 1.5 0.28) (layers F.Cu F.Paste F.Mask) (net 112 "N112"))
  (pad 49 smd rect (at 5.5 7.9 90) (size 1.5 0.28) (layers F.Cu F.Paste F.Mask) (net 6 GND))
  (pad 50 smd rect (at 6 7.9 90) (size 1.5 0.28) (layers F.Cu F.Paste F.Mask) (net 20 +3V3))
  (pad 51 smd rect (at 7.9 6) (size 1.5 0.28) (layers F.Cu F.Paste F.Mask) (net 20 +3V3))
  (pad 52 smd rect (at 7.9 5.5) (size 1.5 0.28) (layers F.Cu F.Paste F.Mask) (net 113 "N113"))
  (pad 53 smd rect (at 7.9 5) (size 1.5 0.28) (layers F.Cu F.Paste F.Mask) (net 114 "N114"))
  (pad 54 smd rect (at 7.9 4.5) (size 1.5 0.28) (layers F.Cu F.Paste F.Mask) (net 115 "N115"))
  (pad 55 smd rect (at 7.9 4) (size 1.5 0.28) (layers F.Cu F.Paste F.Mask) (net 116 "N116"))
  (pad 56 smd rect (at 7.9 3.5) (size 1.5 0.28) (layers F.Cu F.Paste F.Mask) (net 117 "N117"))
  (pad 57 smd rect (at 7.9 3) (size 1.5 0.28) (layers F.Cu F.Paste F.Mask) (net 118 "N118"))
  (pad 58 smd rect (at 7.9 2.5) (size 1.5 0.28) (layers F.Cu F.Paste F.Mask) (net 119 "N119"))
  (pad 59 smd rect (at 7.9 2) (size 1.5 0.28) (layers F.Cu F.Paste F.Mask) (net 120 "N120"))
  (pad 60 smd rect (at 7.9 1.5) (size 1.5 0.28) (layers F.Cu F.Paste F.Mask) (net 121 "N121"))
  (pad 61 smd rect (at 7.9 1) (size 1.5 0.28) (layers F.Cu F.Paste F.Mask) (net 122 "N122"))
  (pad 62 smd rect (at 7.9 0.5) (size 1.5 0.28) (layers F.Cu F.Paste F.Mask) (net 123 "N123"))
  (pad 63 smd rect (at 7.9 0) (size 1.5 0.28) (layers F.Cu F.Paste F.Mask) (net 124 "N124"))
  (pad 64 smd rect (at 7.9 -0.5) (size 1.5 0.28) (layers F.Cu F.Paste F.Mask) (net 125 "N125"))
  (pad 65 smd rect (at 7.9 -1) (size 1.5 0.28) (layers F.Cu F.Paste F.Mask) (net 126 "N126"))
  (pad 66 smd rect (at 7.9 -1.5) (size 1.5 0.28) (layers F.Cu F.Paste F.Mask) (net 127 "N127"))
  (pad 67 smd rect (at 7.9 -2) (size 1.5 0.28) (layers F.Cu F.Paste F.Mask) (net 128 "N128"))
  (pad 68 smd rect (at 7.9 -2.5) (size 1.5 0.28) (layers F.Cu F.Paste F.Mask) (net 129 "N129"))
  (pad 69 smd rect (at 7.9 -3) (size 1.5 0.28) (layers F.Cu F.Paste F.Mask) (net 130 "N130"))
  (pad 70 smd rect (at 7.9 -3.5) (size 1.5 0.28) (layers F.Cu F.Paste F.Mask) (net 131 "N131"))
  (pad 71 smd rect (at 7.9 -4) (size 1.5 0.28) (layers F.Cu F.Paste F.Mask) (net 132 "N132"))
  (pad 72 smd rect (at 7.9 -4.5) (size 1.5 0.28) (layers F.Cu F.Paste F.Mask) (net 67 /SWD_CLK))
  (pad 73 smd rect (at 7.9 -5) (size 1.5 0.28) (layers F.Cu F.Paste F.Mask) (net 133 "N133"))
  (pad 74 smd rect (at 7.9 -5.5) (size 1.5 0.28) (layers F.Cu F.Paste F.Mask) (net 6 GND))
  (pad 75 smd rect (at 7.9 -6) (size 1.5 0.28) (layers F.Cu F.Paste F.Mask) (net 20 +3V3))
  (pad 76 smd rect (at 6 -7.9 90) (size 1.5 0.28) (layers F.Cu F.Paste F.Mask) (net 65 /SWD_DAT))
  (pad 77 smd rect (at 5.5 -7.9 90) (size 1.5 0.28) (layers F.Cu F.Paste F.Mask) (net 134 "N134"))
  (pad 78 smd rect (at 5 -7.9 90) (size 1.5 0.28) (layers F.Cu F.Paste F.Mask) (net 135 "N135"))
  (pad 79 smd rect (at 4.5 -7.9 90) (size 1.5 0.28) (layers F.Cu F.Paste F.Mask) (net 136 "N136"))
  (pad 80 smd rect (at 4 -7.9 90) (size 1.5 0.28) (layers F.Cu F.Paste F.Mask) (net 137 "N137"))
  (pad 81 smd rect (at 3.5 -7.9 90) (size 1.5 0.28) (layers F.Cu F.Paste F.Mask) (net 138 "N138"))
  (pad 82 smd rect (at 3 -7.9 90) (size 1.5 0.28) (layers F.Cu F.Paste F.Mask) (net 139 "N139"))
  (pad 83 smd rect (at 2.5 -7.9 90) (size 1.5 0.28) (layers F.Cu F.Paste F.Mask) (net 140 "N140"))
  (pad 84 smd rect (at 2 -7.9 90) (size 1.5 0.28) (layers F.Cu F.Paste F.Mask) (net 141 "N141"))
  (pad 85 smd rect (at 1.5 -7.9 90) (size 1.5 0.28) (layers F.Cu F.Paste F.Mask) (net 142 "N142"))
  (pad 86 smd rect (at 1 -7.9 90) (size 1.5 0.28) (layers F.Cu F.Paste F.Mask) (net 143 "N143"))
  (pad 87 smd rect (at 0.5 -7.9 90) (size 1.5 0.28) (layers F.Cu F.Paste F.Mask) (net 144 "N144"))
  (pad 88 smd rect (at 0 -7.9 90) (size 1.5 0.28) (layers F.Cu F.Paste F.Mask) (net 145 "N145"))
  (pad 89 smd rect (at -0.5 -7.9 90) (size 1.5 0.28) (layers F.Cu F.Paste F.Mask) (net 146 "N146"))
  (pad 90 smd rect (at -1 -7.9 90) (size 1.5 0.28) (layers F.Cu F.Paste F.Mask) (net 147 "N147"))
  (pad 91 smd rect (at -1.5 -7.9 90) (size 1.5 0.28) (layers F.Cu F.Paste F.Mask) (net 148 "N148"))
  (pad 92 smd rect (at -2 -7.9 90) (size 1.5 0.28) (layers F.Cu F.Paste F.Mask) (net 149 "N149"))
  (pad 93 smd rect (at -2.5 -7.9 90) (size 1.5 0.28) (layers F.Cu F.Paste F.Mask) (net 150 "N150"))
  (pad 94 smd rect (at -3 -7.9 90) (size 1.5 0.28) (layers F.Cu F.Paste F.Mask) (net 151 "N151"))
  (pad 95 smd rect (at -3.5 -7.9 90) (size 1.5 0.28) (layers F.Cu F.Paste F.Mask) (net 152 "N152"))
  (pad 96 smd rect (at -4 -7.9 90) (size 1.5 0.28) (layers F.Cu F.Paste F.Mask) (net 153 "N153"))
  (pad 97 smd rect (at -4.5 -7.9 90) (size 1.5 0.28) (layers F.Cu F.Paste F.Mask) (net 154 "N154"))
  (pad 98 smd rect (at -5 -7.9 90) (size 1.5 0.28) (layers F.Cu F.Paste F.Mask) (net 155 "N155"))
  (pad 99 smd rect (at -5.5 -7.9 90) (size 1.5 0.28) (layers F.Cu F.Paste F.Mask) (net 6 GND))
  (pad 100 smd rect (at -6 -7.9 90) (size 1.5 0.28) (layers F.Cu F.Paste F.Mask) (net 20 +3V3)))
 (gr_line (start 176.53 119.38) (end 125.73 119.38) (layer Edge.Cuts) (width 0.15))
 (gr_line (start 176.53 35.56) (end 176.53 119.38) (layer Edge.Cuts) (width 0.15))
 (gr_line (start 125.73 35.56) (end 176.53 35.56) (layer Edge.Cuts) (width 0.15))
 (gr_line (start 125.73 119.38) (end 125.73 35.56) (layer Edge.Cuts) (width 0.15))
 (segment (start 147.698999 96.094999) (end 147.698999 93.601001) (width 0.25) (layer F.Cu) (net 19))
 (segment (start 148.1075 93.1925) (end 148.1075 91.44) (width 0.25) (layer F.Cu) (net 19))
 (segment (start 147.698999 93.601001) (end 148.1075 93.1925) (width 0.25) (layer F.Cu) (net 19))
 (segment (start 142.618999 96.094999) (end 142.618999 93.088999) (width 0.25) (layer F.Cu) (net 20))
 (segment (start 142.24 92.71) (end 142.24 91.44) (width 0.25) (layer F.Cu) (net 20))
 (segment (start 142.618999 93.088999) (end 142.24 92.71) (width 0.25) (layer F.Cu) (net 20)))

